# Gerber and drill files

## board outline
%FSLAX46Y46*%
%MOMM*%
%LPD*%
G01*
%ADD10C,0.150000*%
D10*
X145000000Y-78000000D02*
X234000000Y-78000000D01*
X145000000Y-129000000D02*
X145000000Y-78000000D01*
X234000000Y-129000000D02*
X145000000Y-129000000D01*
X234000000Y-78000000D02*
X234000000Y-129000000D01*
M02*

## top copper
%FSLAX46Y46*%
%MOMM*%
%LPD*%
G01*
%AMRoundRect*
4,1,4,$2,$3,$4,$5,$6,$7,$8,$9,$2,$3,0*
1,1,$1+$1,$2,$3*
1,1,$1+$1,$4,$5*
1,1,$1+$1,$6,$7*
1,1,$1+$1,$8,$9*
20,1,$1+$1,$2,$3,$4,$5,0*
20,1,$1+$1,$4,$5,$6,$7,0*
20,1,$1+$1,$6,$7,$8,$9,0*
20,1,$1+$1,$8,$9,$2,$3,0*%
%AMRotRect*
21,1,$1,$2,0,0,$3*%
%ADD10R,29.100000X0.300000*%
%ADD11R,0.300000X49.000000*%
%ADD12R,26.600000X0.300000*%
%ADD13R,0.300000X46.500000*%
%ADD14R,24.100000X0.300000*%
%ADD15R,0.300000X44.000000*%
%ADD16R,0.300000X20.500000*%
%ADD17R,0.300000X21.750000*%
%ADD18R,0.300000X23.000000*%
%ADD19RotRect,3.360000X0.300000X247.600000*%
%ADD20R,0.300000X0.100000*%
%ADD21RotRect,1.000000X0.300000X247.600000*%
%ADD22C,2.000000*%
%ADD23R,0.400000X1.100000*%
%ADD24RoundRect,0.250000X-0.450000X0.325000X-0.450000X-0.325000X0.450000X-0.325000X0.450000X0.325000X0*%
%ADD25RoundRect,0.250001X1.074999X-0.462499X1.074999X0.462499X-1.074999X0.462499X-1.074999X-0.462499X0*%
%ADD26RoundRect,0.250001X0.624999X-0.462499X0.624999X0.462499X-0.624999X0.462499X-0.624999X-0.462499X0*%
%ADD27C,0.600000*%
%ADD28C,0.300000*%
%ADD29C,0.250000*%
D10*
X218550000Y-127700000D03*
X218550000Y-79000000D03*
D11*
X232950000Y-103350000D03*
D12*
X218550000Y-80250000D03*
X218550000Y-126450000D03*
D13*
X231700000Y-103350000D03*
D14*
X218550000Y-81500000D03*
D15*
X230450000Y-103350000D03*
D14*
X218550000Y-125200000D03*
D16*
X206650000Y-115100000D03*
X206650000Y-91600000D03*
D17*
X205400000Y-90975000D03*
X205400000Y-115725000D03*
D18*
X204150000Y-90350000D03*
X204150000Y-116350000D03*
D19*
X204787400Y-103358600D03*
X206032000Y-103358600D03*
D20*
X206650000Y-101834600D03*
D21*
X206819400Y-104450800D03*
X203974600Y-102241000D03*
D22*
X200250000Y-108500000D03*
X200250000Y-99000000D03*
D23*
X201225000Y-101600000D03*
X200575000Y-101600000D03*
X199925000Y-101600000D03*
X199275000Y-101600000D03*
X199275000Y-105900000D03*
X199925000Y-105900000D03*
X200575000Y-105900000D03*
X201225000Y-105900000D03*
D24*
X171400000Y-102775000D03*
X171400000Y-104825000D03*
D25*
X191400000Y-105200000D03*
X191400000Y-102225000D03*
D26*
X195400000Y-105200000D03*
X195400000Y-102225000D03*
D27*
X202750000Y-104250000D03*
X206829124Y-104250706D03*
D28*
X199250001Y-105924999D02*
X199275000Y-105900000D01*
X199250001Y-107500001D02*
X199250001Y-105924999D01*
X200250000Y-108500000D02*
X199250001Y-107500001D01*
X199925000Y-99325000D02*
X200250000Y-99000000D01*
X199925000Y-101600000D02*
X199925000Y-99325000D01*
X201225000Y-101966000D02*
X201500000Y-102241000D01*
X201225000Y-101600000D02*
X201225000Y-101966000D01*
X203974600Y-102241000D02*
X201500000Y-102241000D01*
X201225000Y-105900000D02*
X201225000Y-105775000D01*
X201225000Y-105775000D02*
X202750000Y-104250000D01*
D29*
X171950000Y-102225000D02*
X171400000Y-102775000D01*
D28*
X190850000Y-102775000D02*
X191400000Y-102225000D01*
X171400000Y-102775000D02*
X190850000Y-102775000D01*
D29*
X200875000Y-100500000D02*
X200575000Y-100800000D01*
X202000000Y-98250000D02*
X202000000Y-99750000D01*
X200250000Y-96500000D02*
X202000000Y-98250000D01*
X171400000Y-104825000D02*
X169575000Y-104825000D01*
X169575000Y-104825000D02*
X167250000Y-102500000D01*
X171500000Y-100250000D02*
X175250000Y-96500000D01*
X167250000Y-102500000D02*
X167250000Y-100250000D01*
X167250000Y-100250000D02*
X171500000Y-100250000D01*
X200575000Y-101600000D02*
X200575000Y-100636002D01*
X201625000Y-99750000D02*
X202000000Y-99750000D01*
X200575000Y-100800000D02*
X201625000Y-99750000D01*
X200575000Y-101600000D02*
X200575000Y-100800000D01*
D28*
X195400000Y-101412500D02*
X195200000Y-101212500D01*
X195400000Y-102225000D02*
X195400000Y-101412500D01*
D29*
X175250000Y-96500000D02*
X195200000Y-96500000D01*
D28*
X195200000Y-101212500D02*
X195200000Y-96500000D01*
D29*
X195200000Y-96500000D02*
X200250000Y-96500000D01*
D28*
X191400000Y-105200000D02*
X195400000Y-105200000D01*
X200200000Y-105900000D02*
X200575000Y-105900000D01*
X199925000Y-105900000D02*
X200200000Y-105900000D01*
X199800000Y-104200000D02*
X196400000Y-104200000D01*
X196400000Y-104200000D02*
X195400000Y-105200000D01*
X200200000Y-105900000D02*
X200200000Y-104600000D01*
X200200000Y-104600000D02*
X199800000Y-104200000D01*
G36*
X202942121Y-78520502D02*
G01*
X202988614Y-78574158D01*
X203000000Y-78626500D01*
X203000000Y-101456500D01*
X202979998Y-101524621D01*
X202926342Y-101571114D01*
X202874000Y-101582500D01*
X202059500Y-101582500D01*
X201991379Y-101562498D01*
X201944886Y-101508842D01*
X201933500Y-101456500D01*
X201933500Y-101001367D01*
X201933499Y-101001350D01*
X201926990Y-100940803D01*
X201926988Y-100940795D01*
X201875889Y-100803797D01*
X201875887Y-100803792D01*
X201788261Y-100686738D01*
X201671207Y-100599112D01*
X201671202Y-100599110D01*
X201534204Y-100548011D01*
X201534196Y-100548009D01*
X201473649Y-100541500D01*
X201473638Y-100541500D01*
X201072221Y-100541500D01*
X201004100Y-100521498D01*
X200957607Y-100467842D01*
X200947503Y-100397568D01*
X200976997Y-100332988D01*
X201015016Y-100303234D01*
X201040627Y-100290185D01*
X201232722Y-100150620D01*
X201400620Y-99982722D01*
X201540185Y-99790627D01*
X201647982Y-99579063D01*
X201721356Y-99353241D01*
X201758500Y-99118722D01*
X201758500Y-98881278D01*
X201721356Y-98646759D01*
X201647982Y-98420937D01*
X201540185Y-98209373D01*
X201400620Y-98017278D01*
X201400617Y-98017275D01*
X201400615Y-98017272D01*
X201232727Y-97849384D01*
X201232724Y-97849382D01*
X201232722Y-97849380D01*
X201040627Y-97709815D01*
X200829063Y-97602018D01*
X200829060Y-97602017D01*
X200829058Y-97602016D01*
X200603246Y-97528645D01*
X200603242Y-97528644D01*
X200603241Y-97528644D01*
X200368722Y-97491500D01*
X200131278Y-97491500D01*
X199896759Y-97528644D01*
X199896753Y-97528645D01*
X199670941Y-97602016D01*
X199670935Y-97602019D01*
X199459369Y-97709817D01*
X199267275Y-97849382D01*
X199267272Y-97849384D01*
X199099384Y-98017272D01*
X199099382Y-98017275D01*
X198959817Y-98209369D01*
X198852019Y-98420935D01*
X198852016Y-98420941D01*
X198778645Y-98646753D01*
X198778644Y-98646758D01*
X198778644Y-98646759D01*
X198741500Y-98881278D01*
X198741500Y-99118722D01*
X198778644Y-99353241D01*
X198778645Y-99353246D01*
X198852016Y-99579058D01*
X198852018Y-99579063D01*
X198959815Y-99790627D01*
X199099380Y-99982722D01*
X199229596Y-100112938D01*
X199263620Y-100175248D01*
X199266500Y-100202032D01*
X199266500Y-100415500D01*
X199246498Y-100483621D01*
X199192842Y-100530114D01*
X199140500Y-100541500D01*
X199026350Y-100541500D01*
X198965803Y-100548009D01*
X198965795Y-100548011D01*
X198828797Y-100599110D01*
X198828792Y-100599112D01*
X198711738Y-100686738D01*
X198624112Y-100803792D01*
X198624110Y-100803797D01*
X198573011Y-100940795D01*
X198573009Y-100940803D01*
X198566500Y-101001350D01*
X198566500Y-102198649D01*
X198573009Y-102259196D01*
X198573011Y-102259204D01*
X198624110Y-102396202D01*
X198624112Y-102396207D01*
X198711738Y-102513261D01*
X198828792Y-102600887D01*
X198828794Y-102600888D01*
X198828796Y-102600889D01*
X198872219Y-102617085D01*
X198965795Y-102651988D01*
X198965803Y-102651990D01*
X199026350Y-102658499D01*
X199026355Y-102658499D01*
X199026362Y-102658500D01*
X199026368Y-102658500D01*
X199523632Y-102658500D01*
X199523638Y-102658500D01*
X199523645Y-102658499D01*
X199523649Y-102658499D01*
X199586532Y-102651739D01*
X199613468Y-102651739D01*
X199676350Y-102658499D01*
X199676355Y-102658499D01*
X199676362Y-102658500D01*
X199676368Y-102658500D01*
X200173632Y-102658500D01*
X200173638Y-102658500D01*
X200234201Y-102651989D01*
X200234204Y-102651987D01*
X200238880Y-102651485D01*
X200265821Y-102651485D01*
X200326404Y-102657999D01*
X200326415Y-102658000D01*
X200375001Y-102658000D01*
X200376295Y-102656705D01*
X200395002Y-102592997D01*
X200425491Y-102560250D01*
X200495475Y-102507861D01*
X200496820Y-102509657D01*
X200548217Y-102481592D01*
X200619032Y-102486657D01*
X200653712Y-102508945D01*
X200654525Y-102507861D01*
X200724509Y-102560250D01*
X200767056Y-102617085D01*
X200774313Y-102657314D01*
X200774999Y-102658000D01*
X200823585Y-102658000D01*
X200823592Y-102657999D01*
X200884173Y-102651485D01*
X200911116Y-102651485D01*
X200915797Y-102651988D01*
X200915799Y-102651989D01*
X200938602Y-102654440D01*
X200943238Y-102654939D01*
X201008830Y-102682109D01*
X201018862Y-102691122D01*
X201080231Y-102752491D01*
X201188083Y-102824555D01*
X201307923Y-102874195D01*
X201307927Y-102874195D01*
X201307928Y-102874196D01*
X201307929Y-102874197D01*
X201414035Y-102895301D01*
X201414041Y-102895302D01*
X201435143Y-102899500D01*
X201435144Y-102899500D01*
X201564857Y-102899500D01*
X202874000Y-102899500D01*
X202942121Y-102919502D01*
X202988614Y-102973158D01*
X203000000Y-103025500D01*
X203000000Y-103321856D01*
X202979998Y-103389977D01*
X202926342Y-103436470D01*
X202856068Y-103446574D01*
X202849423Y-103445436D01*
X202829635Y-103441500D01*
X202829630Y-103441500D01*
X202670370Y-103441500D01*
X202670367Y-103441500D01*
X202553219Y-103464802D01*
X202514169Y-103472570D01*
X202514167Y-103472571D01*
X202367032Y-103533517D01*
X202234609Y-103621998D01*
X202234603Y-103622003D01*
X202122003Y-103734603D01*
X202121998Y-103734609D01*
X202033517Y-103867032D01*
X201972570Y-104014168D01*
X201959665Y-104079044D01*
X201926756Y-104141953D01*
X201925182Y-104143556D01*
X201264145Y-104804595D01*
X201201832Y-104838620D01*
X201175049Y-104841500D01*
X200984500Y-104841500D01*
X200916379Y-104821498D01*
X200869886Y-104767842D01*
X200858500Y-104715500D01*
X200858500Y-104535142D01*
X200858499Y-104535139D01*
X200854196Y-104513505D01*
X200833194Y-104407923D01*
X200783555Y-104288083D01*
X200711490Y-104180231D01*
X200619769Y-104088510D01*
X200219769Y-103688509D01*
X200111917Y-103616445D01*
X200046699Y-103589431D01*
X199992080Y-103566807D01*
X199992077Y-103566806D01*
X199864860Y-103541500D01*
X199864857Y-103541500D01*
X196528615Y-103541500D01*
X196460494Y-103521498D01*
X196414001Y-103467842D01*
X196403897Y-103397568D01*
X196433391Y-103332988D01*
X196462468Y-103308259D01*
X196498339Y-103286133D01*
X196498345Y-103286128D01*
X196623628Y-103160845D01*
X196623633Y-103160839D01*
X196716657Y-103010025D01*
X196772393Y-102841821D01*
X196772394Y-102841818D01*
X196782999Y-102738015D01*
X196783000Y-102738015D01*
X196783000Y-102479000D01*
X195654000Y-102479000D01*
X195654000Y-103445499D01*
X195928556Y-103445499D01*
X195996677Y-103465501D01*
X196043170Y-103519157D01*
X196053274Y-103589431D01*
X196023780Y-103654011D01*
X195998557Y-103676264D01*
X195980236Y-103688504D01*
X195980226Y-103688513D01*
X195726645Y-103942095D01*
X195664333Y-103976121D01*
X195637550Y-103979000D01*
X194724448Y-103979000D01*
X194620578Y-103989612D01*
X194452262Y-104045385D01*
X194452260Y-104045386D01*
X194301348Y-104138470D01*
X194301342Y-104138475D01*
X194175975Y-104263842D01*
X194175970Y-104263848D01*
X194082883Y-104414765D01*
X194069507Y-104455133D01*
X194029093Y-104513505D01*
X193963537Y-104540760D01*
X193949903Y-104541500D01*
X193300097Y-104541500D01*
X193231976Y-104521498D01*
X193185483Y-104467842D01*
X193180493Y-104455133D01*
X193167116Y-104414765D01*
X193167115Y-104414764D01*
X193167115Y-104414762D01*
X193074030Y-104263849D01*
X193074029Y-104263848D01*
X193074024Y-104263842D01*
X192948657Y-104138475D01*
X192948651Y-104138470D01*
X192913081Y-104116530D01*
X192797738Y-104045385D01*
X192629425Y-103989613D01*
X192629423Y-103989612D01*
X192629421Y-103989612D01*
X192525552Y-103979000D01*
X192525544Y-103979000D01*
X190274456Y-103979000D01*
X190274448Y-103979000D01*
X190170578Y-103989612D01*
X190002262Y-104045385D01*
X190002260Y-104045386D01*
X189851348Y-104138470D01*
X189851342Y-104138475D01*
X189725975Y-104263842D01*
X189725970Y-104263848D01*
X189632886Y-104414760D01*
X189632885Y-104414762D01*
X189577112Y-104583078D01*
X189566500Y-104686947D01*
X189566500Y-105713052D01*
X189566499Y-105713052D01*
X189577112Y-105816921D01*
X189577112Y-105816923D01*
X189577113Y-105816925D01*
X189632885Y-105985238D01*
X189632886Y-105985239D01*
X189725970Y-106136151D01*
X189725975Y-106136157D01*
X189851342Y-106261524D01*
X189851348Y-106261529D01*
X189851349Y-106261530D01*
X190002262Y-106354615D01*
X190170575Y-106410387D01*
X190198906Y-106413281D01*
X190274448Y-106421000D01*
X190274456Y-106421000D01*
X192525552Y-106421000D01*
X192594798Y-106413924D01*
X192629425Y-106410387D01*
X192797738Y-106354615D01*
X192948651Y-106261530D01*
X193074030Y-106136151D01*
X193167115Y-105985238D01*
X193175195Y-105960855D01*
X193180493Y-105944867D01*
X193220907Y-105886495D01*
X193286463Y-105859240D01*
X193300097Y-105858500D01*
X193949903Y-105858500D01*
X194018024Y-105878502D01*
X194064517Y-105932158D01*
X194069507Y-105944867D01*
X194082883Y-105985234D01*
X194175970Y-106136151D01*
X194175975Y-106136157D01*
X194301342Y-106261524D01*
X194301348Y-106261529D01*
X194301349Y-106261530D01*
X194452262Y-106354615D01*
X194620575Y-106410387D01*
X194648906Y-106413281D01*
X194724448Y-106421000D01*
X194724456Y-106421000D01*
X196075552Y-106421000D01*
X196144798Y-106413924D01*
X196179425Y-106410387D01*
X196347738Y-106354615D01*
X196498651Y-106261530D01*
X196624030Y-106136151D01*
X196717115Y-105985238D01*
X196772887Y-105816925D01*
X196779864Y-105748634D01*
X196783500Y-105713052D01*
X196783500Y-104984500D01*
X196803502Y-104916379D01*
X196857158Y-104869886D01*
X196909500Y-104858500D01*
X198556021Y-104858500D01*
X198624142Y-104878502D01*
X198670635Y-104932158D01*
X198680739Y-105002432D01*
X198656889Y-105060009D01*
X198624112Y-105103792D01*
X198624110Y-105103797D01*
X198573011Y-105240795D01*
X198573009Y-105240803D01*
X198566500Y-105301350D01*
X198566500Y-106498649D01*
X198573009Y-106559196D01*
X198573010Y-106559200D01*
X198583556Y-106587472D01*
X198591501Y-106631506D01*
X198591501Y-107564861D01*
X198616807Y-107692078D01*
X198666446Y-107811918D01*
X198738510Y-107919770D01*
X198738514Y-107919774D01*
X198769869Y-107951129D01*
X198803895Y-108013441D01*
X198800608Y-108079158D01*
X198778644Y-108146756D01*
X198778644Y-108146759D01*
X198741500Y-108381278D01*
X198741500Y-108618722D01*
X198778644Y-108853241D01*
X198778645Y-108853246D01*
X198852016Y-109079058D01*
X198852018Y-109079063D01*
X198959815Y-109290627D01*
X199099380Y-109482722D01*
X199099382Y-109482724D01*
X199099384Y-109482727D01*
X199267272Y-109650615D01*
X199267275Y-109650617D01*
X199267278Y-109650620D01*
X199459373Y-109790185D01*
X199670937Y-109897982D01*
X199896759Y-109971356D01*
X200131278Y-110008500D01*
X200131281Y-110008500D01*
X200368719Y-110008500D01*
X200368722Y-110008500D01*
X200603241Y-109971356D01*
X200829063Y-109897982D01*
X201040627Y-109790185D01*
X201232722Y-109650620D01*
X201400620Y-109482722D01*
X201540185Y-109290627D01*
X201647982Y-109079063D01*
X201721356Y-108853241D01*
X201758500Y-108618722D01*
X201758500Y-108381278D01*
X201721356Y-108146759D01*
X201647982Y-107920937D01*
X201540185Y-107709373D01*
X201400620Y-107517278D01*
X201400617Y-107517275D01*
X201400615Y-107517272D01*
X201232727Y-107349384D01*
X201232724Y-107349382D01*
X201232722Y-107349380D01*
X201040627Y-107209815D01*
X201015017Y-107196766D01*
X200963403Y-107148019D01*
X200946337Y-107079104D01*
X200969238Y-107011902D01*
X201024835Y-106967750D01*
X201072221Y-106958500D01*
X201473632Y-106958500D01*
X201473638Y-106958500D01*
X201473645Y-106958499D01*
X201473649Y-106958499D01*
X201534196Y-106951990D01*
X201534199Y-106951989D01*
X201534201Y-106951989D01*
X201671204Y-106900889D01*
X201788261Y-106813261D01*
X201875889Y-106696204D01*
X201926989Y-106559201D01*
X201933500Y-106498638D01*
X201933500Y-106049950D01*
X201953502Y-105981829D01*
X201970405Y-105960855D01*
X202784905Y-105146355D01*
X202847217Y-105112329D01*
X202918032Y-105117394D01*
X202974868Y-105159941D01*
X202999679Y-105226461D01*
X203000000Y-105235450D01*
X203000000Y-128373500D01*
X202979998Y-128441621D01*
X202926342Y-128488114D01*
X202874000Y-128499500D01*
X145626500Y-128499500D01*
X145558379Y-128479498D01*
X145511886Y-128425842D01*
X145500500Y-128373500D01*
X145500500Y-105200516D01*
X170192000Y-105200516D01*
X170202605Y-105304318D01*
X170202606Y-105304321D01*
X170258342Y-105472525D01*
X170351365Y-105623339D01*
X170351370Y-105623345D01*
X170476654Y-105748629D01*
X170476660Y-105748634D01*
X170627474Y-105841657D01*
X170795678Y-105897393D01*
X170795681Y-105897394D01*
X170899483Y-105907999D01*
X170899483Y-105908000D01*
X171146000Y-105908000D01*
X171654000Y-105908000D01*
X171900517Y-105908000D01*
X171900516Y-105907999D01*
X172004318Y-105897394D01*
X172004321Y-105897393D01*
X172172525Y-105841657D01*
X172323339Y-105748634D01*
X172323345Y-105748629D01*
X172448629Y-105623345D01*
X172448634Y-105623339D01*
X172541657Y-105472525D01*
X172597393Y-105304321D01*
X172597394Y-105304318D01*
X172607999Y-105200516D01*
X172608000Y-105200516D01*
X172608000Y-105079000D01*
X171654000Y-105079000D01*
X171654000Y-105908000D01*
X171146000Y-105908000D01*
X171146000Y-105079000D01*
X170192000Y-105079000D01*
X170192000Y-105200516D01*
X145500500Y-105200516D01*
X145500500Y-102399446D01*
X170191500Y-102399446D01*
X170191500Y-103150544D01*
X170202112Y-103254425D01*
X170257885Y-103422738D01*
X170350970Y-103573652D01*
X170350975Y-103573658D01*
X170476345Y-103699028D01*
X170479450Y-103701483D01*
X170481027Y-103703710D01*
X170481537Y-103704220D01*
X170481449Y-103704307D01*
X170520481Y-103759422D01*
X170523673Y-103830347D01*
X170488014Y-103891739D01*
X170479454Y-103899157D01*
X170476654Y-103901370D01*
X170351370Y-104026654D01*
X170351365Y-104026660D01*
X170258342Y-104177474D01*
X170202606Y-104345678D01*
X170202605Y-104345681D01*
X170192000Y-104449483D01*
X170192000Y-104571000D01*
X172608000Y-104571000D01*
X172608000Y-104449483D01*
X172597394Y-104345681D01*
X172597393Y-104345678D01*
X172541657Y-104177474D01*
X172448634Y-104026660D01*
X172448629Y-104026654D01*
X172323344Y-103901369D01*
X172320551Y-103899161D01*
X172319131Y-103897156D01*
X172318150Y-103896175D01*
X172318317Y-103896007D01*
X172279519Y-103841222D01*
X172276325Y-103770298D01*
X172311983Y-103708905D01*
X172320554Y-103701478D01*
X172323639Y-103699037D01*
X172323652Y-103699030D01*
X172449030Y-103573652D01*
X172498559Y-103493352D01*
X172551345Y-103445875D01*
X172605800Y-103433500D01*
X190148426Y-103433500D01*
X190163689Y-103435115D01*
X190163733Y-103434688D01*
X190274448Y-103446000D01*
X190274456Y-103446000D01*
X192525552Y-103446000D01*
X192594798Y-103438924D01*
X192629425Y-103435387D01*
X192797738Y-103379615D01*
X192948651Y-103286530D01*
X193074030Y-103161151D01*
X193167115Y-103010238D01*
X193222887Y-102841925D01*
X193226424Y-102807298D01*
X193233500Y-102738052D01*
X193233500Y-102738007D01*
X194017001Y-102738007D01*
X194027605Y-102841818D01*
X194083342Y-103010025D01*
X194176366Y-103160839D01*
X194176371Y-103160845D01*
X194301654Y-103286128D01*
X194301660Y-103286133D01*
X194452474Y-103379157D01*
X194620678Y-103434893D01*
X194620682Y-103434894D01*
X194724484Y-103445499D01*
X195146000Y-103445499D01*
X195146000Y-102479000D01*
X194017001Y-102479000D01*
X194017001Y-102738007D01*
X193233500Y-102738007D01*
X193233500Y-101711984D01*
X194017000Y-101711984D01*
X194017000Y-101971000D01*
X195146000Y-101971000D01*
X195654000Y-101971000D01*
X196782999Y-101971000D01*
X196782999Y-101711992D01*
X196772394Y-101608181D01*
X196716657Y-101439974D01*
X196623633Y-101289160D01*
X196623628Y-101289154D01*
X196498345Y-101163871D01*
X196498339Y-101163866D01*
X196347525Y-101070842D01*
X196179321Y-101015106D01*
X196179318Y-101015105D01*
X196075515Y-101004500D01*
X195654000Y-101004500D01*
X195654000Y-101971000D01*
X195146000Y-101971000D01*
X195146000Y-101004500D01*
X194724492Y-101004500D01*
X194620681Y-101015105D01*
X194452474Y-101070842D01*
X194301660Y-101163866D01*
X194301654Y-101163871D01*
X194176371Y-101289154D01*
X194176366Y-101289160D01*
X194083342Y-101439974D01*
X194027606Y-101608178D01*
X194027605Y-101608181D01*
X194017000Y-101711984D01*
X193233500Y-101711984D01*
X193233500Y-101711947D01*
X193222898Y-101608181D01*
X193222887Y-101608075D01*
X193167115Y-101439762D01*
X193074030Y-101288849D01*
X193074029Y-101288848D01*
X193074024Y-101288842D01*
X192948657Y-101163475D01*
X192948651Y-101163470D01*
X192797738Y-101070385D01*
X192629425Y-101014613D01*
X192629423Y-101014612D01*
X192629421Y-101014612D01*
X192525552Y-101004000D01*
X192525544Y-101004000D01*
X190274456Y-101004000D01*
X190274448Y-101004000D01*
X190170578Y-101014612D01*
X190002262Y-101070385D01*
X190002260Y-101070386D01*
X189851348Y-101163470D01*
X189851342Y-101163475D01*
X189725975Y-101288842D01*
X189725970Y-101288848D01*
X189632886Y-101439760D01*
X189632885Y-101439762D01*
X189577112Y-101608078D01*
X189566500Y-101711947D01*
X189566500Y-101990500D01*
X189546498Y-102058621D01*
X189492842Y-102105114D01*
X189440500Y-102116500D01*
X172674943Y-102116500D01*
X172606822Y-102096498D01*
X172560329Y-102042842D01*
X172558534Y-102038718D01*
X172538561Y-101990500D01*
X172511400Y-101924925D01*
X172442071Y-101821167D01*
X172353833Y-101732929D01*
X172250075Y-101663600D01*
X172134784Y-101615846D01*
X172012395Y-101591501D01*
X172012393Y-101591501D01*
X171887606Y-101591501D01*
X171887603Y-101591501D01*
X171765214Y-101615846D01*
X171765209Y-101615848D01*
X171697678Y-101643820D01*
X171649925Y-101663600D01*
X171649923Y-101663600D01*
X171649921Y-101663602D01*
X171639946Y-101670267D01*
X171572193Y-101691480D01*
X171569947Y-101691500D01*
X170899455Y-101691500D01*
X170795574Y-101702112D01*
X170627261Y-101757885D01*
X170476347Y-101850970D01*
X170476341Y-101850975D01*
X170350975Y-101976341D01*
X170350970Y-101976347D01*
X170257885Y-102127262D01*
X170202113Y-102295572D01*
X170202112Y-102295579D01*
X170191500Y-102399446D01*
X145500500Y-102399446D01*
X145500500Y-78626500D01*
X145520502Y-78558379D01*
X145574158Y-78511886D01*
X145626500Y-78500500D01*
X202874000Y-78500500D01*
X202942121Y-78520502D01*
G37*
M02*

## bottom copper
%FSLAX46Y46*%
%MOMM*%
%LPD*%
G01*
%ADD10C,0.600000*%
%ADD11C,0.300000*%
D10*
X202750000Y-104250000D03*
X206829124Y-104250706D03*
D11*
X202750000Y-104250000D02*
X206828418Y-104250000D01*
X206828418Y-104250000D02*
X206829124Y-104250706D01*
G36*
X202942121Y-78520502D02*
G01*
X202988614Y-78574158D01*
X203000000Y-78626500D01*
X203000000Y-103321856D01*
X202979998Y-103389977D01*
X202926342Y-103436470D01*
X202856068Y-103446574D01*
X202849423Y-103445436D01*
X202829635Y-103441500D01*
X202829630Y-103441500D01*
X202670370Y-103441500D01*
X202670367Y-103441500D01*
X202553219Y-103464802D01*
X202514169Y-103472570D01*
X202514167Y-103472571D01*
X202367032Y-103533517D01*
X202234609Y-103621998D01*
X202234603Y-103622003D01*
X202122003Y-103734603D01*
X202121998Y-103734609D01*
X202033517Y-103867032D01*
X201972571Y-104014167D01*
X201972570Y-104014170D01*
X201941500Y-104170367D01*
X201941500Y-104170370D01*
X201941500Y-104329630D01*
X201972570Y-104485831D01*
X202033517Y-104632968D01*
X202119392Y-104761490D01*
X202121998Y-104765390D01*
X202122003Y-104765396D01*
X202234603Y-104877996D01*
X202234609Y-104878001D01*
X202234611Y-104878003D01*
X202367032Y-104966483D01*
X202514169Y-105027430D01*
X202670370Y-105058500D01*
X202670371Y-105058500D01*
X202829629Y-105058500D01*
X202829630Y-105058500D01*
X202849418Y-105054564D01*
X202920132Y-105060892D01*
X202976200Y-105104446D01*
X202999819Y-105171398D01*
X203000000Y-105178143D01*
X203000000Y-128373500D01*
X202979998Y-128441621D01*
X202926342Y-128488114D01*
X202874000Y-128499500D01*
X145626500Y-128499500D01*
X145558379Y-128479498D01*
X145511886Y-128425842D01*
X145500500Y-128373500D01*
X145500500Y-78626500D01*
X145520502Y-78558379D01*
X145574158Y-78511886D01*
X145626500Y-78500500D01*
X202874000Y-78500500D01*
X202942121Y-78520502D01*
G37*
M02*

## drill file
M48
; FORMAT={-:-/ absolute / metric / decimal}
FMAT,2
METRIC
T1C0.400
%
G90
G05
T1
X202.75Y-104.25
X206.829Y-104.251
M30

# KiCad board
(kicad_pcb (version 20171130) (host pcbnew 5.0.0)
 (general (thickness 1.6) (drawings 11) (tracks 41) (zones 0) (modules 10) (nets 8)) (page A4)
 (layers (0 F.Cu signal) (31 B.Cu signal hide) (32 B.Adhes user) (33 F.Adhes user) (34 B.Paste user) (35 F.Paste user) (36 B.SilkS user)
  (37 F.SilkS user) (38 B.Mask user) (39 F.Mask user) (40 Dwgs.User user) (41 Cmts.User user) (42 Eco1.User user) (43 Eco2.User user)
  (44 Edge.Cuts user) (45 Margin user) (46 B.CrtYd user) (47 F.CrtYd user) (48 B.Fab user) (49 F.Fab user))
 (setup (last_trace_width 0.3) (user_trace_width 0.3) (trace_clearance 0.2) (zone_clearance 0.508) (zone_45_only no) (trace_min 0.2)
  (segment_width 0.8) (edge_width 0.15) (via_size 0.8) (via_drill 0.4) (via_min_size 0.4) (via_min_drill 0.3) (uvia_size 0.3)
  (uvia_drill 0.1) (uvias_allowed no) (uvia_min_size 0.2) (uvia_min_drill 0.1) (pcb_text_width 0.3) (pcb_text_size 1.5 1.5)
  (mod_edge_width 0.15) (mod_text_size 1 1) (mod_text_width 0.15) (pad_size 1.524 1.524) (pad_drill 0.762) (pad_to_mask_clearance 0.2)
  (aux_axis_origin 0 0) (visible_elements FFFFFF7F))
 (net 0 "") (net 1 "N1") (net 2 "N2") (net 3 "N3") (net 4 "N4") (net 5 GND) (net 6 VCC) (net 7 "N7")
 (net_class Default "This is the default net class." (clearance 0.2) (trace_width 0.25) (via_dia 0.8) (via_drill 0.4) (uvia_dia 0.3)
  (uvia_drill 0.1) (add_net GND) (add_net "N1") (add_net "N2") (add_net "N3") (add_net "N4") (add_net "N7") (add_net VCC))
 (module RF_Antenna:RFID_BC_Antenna (layer F.Cu) (at 204 79)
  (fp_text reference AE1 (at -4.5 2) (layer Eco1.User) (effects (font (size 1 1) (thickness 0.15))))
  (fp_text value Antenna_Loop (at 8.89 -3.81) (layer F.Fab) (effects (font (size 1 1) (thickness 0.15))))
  (pad 1 smd rect (at 14.55 48.7) (size 29.1 0.3) (layers F.Cu F.Paste) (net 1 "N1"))
  (pad 1 smd rect (at 14.55 0) (size 29.1 0.3) (layers F.Cu F.Paste) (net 1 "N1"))
  (pad 2 smd rect (at 28.95 24.35 90) (size 49 0.3) (layers F.Cu F.Paste) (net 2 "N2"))
  (pad 1 smd rect (at 14.55 1.25) (size 26.6 0.3) (layers F.Cu F.Paste) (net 1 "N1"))
  (pad 1 smd rect (at 14.55 47.45) (size 26.6 0.3) (layers F.Cu F.Paste) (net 1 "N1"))
  (pad 1 smd rect (at 27.7 24.35 90) (size 46.5 0.3) (layers F.Cu F.Paste) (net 1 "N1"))
  (pad 1 smd rect (at 14.55 2.5) (size 24.1 0.3) (layers F.Cu F.Paste) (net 1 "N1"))
  (pad 1 smd rect (at 26.45 24.35 90) (size 44 0.3) (layers F.Cu F.Paste) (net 1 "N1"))
  (pad 1 smd rect (at 14.55 46.2) (size 24.1 0.3) (layers F.Cu F.Paste) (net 1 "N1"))
  (pad 1 smd rect (at 2.65 36.1 90) (size 20.5 0.3) (layers F.Cu F.Paste) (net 1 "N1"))
  (pad 1 smd rect (at 2.65 12.6 90) (size 20.5 0.3) (layers F.Cu F.Paste) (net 1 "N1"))
  (pad 1 smd rect (at 1.4 11.975 90) (size 21.75 0.3) (layers F.Cu F.Paste) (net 1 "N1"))
  (pad 1 smd rect (at 1.4 36.725 90) (size 21.75 0.3) (layers F.Cu F.Paste) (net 1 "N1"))
  (pad 1 smd rect (at 0.15 11.35 90) (size 23 0.3) (layers F.Cu F.Paste) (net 1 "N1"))
  (pad 1 smd rect (at 0.15 37.35 90) (size 23 0.3) (layers F.Cu F.Paste) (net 1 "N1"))
  (pad 1 smd rect (at 0.7874 24.3586 247.6) (size 3.36 0.3) (layers F.Cu F.Paste) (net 1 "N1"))
  (pad 1 smd rect (at 2.032 24.3586 247.6) (size 3.36 0.3) (layers F.Cu F.Paste) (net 1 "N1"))
  (pad 1 smd rect (at 2.65 22.8346 90) (size 0.1 0.3) (layers F.Cu F.Paste) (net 1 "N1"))
  (pad 2 smd rect (at 2.8194 25.4508 247.6) (size 1 0.3) (layers F.Cu F.Paste F.Mask) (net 2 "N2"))
  (pad 1 smd rect (at -0.0254 23.241 247.6) (size 1 0.3) (layers F.Cu F.Paste F.Mask) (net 1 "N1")))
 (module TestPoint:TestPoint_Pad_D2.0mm (layer F.Cu) (at 200.25 108.5)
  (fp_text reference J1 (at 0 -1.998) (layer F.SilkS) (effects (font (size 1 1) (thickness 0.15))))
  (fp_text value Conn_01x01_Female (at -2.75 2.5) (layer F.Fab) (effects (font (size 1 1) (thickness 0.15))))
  (pad 1 smd circle (at 0 0) (size 2 2) (layers F.Cu F.Mask) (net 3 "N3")))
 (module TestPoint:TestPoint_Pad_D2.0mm (layer F.Cu) (at 200.25 99)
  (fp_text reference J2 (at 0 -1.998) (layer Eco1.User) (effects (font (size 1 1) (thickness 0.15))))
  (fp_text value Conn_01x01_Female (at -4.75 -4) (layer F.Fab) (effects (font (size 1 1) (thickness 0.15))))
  (pad 1 smd circle (at 0 0) (size 2 2) (layers F.Cu F.Mask) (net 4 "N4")))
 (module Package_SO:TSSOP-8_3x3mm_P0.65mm (layer F.Cu) (at 200.25 103.75 270)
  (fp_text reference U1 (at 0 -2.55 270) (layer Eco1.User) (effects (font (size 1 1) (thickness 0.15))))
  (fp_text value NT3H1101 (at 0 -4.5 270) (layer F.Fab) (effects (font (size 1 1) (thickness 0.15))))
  (pad 1 smd rect (at -2.15 -0.975 270) (size 1.1 0.4) (layers F.Cu F.Paste F.Mask) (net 1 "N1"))
  (pad 2 smd rect (at -2.15 -0.325 270) (size 1.1 0.4) (layers F.Cu F.Paste F.Mask) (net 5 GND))
  (pad 3 smd rect (at -2.15 0.325 270) (size 1.1 0.4) (layers F.Cu F.Paste F.Mask) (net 4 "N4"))
  (pad 4 smd rect (at -2.15 0.975 270) (size 1.1 0.4) (layers F.Cu F.Paste F.Mask))
  (pad 5 smd rect (at 2.15 0.975 270) (size 1.1 0.4) (layers F.Cu F.Paste F.Mask) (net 3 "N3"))
  (pad 6 smd rect (at 2.15 0.325 270) (size 1.1 0.4) (layers F.Cu F.Paste F.Mask) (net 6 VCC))
  (pad 7 smd rect (at 2.15 -0.325 270) (size 1.1 0.4) (layers F.Cu F.Paste F.Mask) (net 6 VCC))
  (pad 8 smd rect (at 2.15 -0.975 270) (size 1.1 0.4) (layers F.Cu F.Paste F.Mask) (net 2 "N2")))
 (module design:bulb (layer F.Cu) (at 173.8 103.4 90)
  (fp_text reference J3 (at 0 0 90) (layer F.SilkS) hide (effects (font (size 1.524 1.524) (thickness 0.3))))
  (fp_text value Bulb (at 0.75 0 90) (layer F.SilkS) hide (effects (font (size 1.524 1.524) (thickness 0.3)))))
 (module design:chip (layer B.Cu) (at 152.75 85.25)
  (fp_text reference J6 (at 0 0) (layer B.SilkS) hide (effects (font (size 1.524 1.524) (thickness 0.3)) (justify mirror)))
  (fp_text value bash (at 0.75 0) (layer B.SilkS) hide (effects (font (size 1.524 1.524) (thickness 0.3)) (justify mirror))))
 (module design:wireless (layer F.Cu) (at 220 102.4)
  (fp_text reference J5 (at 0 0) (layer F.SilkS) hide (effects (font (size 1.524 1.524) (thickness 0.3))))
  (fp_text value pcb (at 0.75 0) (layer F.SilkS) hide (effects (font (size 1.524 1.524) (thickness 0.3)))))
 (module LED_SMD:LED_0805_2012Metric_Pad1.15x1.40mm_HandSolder (layer F.Cu) (at 171.4 103.8 270)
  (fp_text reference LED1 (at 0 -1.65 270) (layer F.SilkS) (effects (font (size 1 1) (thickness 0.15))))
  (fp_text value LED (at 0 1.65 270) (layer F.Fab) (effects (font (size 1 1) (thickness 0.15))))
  (pad 1 smd roundrect (at -1.025 0 270) (size 1.15 1.4) (layers F.Cu F.Paste F.Mask) (roundrect_rratio 0.217391) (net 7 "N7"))
  (pad 2 smd roundrect (at 1.025 0 270) (size 1.15 1.4) (layers F.Cu F.Paste F.Mask) (roundrect_rratio 0.217391) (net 5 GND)))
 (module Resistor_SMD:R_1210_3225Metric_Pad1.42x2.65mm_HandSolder (layer F.Cu) (at 191.4 103.7125 90)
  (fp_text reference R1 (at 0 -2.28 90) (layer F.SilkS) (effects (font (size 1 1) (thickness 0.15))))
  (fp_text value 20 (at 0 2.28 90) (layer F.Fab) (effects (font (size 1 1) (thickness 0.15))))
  (pad 1 smd roundrect (at -1.4875 0 90) (size 1.425 2.65) (layers F.Cu F.Paste F.Mask) (roundrect_rratio 0.175439) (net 6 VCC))
  (pad 2 smd roundrect (at 1.4875 0 90) (size 1.425 2.65) (layers F.Cu F.Paste F.Mask) (roundrect_rratio 0.175439) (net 7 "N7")))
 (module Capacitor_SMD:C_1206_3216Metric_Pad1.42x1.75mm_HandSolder (layer F.Cu) (at 195.4 103.7125 90)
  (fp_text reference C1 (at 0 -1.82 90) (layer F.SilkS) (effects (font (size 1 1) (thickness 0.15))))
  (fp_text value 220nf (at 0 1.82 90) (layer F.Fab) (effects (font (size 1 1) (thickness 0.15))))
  (pad 1 smd roundrect (at -1.4875 0 90) (size 1.425 1.75) (layers F.Cu F.Paste F.Mask) (roundrect_rratio 0.175439) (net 6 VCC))
  (pad 2 smd roundrect (at 1.4875 0 90) (size 1.425 1.75) (layers F.Cu F.Paste F.Mask) (roundrect_rratio 0.175439) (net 5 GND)))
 (gr_line (start 145 78) (end 234 78) (layer Edge.Cuts) (width 0.15))
 (gr_line (start 145 129) (end 145 78) (layer Edge.Cuts) (width 0.15))
 (gr_line (start 234 129) (end 145 129) (layer Edge.Cuts) (width 0.15))
 (gr_line (start 234 78) (end 234 129) (layer Edge.Cuts) (width 0.15))
 (segment (start 199.250001 105.924999) (end 199.275 105.9) (width 0.3) (layer F.Cu) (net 3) (status 30))
 (segment (start 199.250001 107.500001) (end 199.250001 105.924999) (width 0.3) (layer F.Cu) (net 3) (status 20))
 (segment (start 200.25 108.5) (end 199.250001 107.500001) (width 0.3) (layer F.Cu) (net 3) (status 10))
 (segment (start 199.925 99.325) (end 200.25 99) (width 0.3) (layer F.Cu) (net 4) (status 30))
 (segment (start 199.925 101.6) (end 199.925 99.325) (width 0.3) (layer F.Cu) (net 4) (status 30))
 (segment (start 201.225 101.966) (end 201.5 102.241) (width 0.3) (layer F.Cu) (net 1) (status 10))
 (segment (start 201.225 101.6) (end 201.225 101.966) (width 0.3) (layer F.Cu) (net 1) (status 30))
 (segment (start 203.9746 102.241) (end 201.5 102.241) (width 0.3) (layer F.Cu) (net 1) (status 10))
 (via (at 202.75 104.25) (size 0.6) (drill 0.4) (layers F.Cu B.Cu) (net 2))
 (segment (start 201.225 105.9) (end 201.225 105.775) (width 0.3) (layer F.Cu) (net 2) (status 30))
 (segment (start 201.225 105.775) (end 202.75 104.25) (width 0.3) (layer F.Cu) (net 2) (status 10))
 (via (at 206.829124 104.250706) (size 0.6) (drill 0.4) (layers F.Cu B.Cu) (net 2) (status 30))
 (segment (start 202.75 104.25) (end 206.828418 104.25) (width 0.3) (layer B.Cu) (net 2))
 (segment (start 206.828418 104.25) (end 206.829124 104.250706) (width 0.3) (layer B.Cu) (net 2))
 (segment (start 171.95 102.225) (end 171.4 102.775) (width 0.25) (layer F.Cu) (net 7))
 (segment (start 190.85 102.775) (end 191.4 102.225) (width 0.3) (layer F.Cu) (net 7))
 (segment (start 171.4 102.775) (end 190.85 102.775) (width 0.3) (layer F.Cu) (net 7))
 (segment (start 200.875 100.5) (end 200.575 100.8) (width 0.25) (layer F.Cu) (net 5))
 (segment (start 202 98.25) (end 202 99.75) (width 0.25) (layer F.Cu) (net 5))
 (segment (start 200.25 96.5) (end 202 98.25) (width 0.25) (layer F.Cu) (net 5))
 (segment (start 171.4 104.825) (end 169.575 104.825) (width 0.25) (layer F.Cu) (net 5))
 (segment (start 169.575 104.825) (end 167.25 102.5) (width 0.25) (layer F.Cu) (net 5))
 (segment (start 171.5 100.25) (end 175.25 96.5) (width 0.25) (layer F.Cu) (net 5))
 (segment (start 167.25 102.5) (end 167.25 100.25) (width 0.25) (layer F.Cu) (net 5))
 (segment (start 167.25 100.25) (end 171.5 100.25) (width 0.25) (layer F.Cu) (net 5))
 (segment (start 200.575 101.6) (end 200.575 100.636002) (width 0.25) (layer F.Cu) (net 5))
 (segment (start 201.625 99.75) (end 202 99.75) (width 0.25) (layer F.Cu) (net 5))
 (segment (start 200.575 100.8) (end 201.625 99.75) (width 0.25) (layer F.Cu) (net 5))
 (segment (start 200.575 101.6) (end 200.575 100.8) (width 0.25) (layer F.Cu) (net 5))
 (segment (start 195.4 101.4125) (end 195.2 101.2125) (width 0.3) (layer F.Cu) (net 5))
 (segment (start 195.4 102.225) (end 195.4 101.4125) (width 0.3) (layer F.Cu) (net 5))
 (segment (start 175.25 96.5) (end 195.2 96.5) (width 0.25) (layer F.Cu) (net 5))
 (segment (start 195.2 101.2125) (end 195.2 96.5) (width 0.3) (layer F.Cu) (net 5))
 (segment (start 195.2 96.5) (end 200.25 96.5) (width 0.25) (layer F.Cu) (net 5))
 (segment (start 191.4 105.2) (end 195.4 105.2) (width 0.3) (layer F.Cu) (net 6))
 (segment (start 200.2 105.9) (end 200.575 105.9) (width 0.3) (layer F.Cu) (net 6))
 (segment (start 199.925 105.9) (end 200.2 105.9) (width 0.3) (layer F.Cu) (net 6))
 (segment (start 199.8 104.2) (end 196.4 104.2) (width 0.3) (layer F.Cu) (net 6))
 (segment (start 196.4 104.2) (end 195.4 105.2) (width 0.3) (layer F.Cu) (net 6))
 (segment (start 200.2 105.9) (end 200.2 104.6) (width 0.3) (layer F.Cu) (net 6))
 (segment (start 200.2 104.6) (end 199.8 104.2) (width 0.3) (layer F.Cu) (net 6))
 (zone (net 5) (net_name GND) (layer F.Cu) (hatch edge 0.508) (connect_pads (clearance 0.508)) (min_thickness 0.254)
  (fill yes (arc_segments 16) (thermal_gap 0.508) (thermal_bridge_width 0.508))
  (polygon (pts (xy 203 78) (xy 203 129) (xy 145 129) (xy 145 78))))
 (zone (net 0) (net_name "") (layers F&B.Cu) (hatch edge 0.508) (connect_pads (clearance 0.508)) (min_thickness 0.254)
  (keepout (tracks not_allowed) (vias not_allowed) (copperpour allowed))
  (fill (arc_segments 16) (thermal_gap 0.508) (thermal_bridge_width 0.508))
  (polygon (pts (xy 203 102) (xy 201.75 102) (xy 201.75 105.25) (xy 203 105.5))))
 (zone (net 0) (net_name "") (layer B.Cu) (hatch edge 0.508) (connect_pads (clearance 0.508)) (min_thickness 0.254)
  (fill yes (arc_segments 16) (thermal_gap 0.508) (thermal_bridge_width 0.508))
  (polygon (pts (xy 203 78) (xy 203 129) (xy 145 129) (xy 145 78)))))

